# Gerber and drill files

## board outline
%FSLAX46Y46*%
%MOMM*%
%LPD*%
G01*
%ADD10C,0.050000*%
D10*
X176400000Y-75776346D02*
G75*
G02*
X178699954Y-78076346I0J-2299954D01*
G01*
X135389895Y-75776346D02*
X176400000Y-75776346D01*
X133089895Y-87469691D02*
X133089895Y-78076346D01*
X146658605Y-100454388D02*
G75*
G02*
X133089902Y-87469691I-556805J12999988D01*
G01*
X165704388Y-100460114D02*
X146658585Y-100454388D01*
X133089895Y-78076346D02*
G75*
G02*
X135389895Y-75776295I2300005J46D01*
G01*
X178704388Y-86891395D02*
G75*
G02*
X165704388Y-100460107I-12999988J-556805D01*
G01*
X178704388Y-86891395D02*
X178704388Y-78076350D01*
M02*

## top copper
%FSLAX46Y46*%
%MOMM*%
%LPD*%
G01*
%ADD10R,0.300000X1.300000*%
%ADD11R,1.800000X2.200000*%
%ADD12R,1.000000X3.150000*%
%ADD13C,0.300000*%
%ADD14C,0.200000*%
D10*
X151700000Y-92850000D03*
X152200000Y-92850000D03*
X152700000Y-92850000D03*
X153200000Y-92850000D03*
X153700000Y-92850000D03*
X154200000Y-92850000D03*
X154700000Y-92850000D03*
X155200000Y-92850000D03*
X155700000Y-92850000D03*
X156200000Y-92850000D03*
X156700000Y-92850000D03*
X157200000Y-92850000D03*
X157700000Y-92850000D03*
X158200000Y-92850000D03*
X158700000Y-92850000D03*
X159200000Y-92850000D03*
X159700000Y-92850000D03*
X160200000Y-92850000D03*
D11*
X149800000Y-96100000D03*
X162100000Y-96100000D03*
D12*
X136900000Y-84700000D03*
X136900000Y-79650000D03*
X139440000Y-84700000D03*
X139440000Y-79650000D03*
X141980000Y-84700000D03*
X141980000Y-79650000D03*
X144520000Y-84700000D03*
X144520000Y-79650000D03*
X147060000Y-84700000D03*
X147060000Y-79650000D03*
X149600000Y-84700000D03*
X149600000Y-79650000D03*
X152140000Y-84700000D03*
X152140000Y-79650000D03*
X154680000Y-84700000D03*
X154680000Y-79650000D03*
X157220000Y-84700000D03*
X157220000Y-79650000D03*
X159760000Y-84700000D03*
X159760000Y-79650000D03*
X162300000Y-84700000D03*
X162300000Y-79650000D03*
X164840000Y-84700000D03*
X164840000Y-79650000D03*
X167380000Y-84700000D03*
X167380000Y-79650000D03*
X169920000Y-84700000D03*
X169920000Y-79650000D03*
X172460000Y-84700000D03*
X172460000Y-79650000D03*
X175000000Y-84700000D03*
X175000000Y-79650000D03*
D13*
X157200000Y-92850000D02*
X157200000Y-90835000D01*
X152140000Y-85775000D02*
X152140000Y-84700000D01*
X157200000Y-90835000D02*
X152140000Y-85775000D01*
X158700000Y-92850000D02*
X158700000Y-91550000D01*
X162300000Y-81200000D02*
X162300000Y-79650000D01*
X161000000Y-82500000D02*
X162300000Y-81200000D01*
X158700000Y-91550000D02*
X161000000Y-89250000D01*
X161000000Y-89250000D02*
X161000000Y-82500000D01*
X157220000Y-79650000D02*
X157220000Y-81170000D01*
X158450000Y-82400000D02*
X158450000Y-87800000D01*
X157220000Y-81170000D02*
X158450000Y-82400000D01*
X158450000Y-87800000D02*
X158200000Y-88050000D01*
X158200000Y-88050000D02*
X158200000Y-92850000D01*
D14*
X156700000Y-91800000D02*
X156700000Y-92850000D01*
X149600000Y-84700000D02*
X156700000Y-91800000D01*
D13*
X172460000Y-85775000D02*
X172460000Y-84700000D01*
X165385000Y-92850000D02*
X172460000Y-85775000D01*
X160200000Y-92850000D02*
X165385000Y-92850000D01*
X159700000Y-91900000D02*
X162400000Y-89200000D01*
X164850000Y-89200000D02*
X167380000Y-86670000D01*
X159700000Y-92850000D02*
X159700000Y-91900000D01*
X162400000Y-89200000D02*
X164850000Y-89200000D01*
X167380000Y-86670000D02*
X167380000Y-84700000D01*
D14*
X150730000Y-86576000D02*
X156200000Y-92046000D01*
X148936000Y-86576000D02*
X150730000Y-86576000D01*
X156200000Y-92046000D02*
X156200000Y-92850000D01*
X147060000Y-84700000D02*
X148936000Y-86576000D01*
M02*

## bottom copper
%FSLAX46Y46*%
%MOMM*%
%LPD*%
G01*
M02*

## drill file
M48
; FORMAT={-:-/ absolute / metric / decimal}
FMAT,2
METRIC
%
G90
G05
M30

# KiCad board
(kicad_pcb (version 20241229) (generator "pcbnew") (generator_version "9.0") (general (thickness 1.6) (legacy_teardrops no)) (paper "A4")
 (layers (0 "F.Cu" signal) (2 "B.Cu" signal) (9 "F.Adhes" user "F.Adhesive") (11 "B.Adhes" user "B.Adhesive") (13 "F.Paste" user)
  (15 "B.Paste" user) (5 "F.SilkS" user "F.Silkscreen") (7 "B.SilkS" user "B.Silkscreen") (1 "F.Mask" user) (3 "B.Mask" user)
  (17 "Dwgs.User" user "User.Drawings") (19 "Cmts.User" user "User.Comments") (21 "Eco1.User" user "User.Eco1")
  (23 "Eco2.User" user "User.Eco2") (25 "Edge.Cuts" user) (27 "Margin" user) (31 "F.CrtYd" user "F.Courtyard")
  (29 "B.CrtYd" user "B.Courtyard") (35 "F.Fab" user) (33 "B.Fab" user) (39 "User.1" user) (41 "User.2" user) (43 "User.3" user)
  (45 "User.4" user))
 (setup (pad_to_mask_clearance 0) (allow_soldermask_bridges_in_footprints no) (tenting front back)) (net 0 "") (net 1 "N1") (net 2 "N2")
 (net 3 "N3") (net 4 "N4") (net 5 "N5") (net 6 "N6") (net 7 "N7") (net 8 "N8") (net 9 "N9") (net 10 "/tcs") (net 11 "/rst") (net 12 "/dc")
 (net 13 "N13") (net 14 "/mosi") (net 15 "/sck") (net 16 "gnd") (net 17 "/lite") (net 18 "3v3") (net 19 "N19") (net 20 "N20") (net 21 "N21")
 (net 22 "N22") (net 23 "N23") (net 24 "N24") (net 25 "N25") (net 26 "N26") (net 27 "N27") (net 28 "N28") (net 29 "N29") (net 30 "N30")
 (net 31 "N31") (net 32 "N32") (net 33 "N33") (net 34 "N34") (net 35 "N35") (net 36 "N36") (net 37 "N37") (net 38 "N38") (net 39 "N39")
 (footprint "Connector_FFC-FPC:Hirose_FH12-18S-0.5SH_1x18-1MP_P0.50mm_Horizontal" (layer "F.Cu") (at 155.95 94.7)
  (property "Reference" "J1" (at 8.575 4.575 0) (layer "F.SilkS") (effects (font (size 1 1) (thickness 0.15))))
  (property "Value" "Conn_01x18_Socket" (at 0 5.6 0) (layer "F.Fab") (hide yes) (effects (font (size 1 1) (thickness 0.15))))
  (pad "1" smd rect (at -4.25 -1.85) (size 0.3 1.3) (layers "F.Cu" "F.Mask" "F.Paste") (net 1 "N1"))
  (pad "2" smd rect (at -3.75 -1.85) (size 0.3 1.3) (layers "F.Cu" "F.Mask" "F.Paste") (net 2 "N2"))
  (pad "3" smd rect (at -3.25 -1.85) (size 0.3 1.3) (layers "F.Cu" "F.Mask" "F.Paste") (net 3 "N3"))
  (pad "4" smd rect (at -2.75 -1.85) (size 0.3 1.3) (layers "F.Cu" "F.Mask" "F.Paste") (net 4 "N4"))
  (pad "5" smd rect (at -2.25 -1.85) (size 0.3 1.3) (layers "F.Cu" "F.Mask" "F.Paste") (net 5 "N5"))
  (pad "6" smd rect (at -1.75 -1.85) (size 0.3 1.3) (layers "F.Cu" "F.Mask" "F.Paste") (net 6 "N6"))
  (pad "7" smd rect (at -1.25 -1.85) (size 0.3 1.3) (layers "F.Cu" "F.Mask" "F.Paste") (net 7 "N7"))
  (pad "8" smd rect (at -0.75 -1.85) (size 0.3 1.3) (layers "F.Cu" "F.Mask" "F.Paste") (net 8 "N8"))
  (pad "9" smd rect (at -0.25 -1.85) (size 0.3 1.3) (layers "F.Cu" "F.Mask" "F.Paste") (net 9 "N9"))
  (pad "10" smd rect (at 0.25 -1.85) (size 0.3 1.3) (layers "F.Cu" "F.Mask" "F.Paste") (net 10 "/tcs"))
  (pad "11" smd rect (at 0.75 -1.85) (size 0.3 1.3) (layers "F.Cu" "F.Mask" "F.Paste") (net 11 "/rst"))
  (pad "12" smd rect (at 1.25 -1.85) (size 0.3 1.3) (layers "F.Cu" "F.Mask" "F.Paste") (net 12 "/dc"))
  (pad "13" smd rect (at 1.75 -1.85) (size 0.3 1.3) (layers "F.Cu" "F.Mask" "F.Paste") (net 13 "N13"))
  (pad "14" smd rect (at 2.25 -1.85) (size 0.3 1.3) (layers "F.Cu" "F.Mask" "F.Paste") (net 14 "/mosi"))
  (pad "15" smd rect (at 2.75 -1.85) (size 0.3 1.3) (layers "F.Cu" "F.Mask" "F.Paste") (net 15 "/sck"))
  (pad "16" smd rect (at 3.25 -1.85) (size 0.3 1.3) (layers "F.Cu" "F.Mask" "F.Paste") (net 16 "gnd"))
  (pad "17" smd rect (at 3.75 -1.85) (size 0.3 1.3) (layers "F.Cu" "F.Mask" "F.Paste") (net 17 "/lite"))
  (pad "18" smd rect (at 4.25 -1.85) (size 0.3 1.3) (layers "F.Cu" "F.Mask" "F.Paste") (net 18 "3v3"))
  (pad "MP" smd rect (at -6.15 1.4) (size 1.8 2.2) (layers "F.Cu" "F.Mask" "F.Paste"))
  (pad "MP" smd rect (at 6.15 1.4) (size 1.8 2.2) (layers "F.Cu" "F.Mask" "F.Paste")))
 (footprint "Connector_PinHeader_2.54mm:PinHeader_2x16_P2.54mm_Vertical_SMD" (layer "F.Cu") (at 155.95 82.175 90)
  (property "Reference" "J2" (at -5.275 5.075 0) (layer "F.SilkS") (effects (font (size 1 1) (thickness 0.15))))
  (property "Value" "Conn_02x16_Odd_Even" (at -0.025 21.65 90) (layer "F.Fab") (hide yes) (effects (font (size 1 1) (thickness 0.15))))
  (pad "1" smd rect (at -2.525 -19.05 90) (size 3.15 1) (layers "F.Cu" "F.Mask" "F.Paste") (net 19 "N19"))
  (pad "2" smd rect (at 2.525 -19.05 90) (size 3.15 1) (layers "F.Cu" "F.Mask" "F.Paste") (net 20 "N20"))
  (pad "3" smd rect (at -2.525 -16.51 90) (size 3.15 1) (layers "F.Cu" "F.Mask" "F.Paste") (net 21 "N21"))
  (pad "4" smd rect (at 2.525 -16.51 90) (size 3.15 1) (layers "F.Cu" "F.Mask" "F.Paste") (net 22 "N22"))
  (pad "5" smd rect (at -2.525 -13.97 90) (size 3.15 1) (layers "F.Cu" "F.Mask" "F.Paste") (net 16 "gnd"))
  (pad "6" smd rect (at 2.525 -13.97 90) (size 3.15 1) (layers "F.Cu" "F.Mask" "F.Paste") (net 16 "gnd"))
  (pad "7" smd rect (at -2.525 -11.43 90) (size 3.15 1) (layers "F.Cu" "F.Mask" "F.Paste") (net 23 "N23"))
  (pad "8" smd rect (at 2.525 -11.43 90) (size 3.15 1) (layers "F.Cu" "F.Mask" "F.Paste") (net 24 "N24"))
  (pad "9" smd rect (at -2.525 -8.89 90) (size 3.15 1) (layers "F.Cu" "F.Mask" "F.Paste") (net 10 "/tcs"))
  (pad "10" smd rect (at 2.525 -8.89 90) (size 3.15 1) (layers "F.Cu" "F.Mask" "F.Paste") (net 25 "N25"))
  (pad "11" smd rect (at -2.525 -6.35 90) (size 3.15 1) (layers "F.Cu" "F.Mask" "F.Paste") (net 11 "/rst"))
  (pad "12" smd rect (at 2.525 -6.35 90) (size 3.15 1) (layers "F.Cu" "F.Mask" "F.Paste") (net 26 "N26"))
  (pad "13" smd rect (at -2.525 -3.81 90) (size 3.15 1) (layers "F.Cu" "F.Mask" "F.Paste") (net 12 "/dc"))
  (pad "14" smd rect (at 2.525 -3.81 90) (size 3.15 1) (layers "F.Cu" "F.Mask" "F.Paste") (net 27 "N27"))
  (pad "15" smd rect (at -2.525 -1.27 90) (size 3.15 1) (layers "F.Cu" "F.Mask" "F.Paste") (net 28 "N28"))
  (pad "16" smd rect (at 2.525 -1.27 90) (size 3.15 1) (layers "F.Cu" "F.Mask" "F.Paste") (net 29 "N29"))
  (pad "17" smd rect (at -2.525 1.27 90) (size 3.15 1) (layers "F.Cu" "F.Mask" "F.Paste") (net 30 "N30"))
  (pad "18" smd rect (at 2.525 1.27 90) (size 3.15 1) (layers "F.Cu" "F.Mask" "F.Paste") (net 14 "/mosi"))
  (pad "19" smd rect (at -2.525 3.81 90) (size 3.15 1) (layers "F.Cu" "F.Mask" "F.Paste") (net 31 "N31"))
  (pad "20" smd rect (at 2.525 3.81 90) (size 3.15 1) (layers "F.Cu" "F.Mask" "F.Paste") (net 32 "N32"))
  (pad "21" smd rect (at -2.525 6.35 90) (size 3.15 1) (layers "F.Cu" "F.Mask" "F.Paste") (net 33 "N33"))
  (pad "22" smd rect (at 2.525 6.35 90) (size 3.15 1) (layers "F.Cu" "F.Mask" "F.Paste") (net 15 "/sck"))
  (pad "23" smd rect (at -2.525 8.89 90) (size 3.15 1) (layers "F.Cu" "F.Mask" "F.Paste") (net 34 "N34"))
  (pad "24" smd rect (at 2.525 8.89 90) (size 3.15 1) (layers "F.Cu" "F.Mask" "F.Paste") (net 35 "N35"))
  (pad "25" smd rect (at -2.525 11.43 90) (size 3.15 1) (layers "F.Cu" "F.Mask" "F.Paste") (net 17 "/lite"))
  (pad "26" smd rect (at 2.525 11.43 90) (size 3.15 1) (layers "F.Cu" "F.Mask" "F.Paste") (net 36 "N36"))
  (pad "27" smd rect (at -2.525 13.97 90) (size 3.15 1) (layers "F.Cu" "F.Mask" "F.Paste") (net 16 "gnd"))
  (pad "28" smd rect (at 2.525 13.97 90) (size 3.15 1) (layers "F.Cu" "F.Mask" "F.Paste") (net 16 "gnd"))
  (pad "29" smd rect (at -2.525 16.51 90) (size 3.15 1) (layers "F.Cu" "F.Mask" "F.Paste") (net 18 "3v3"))
  (pad "30" smd rect (at 2.525 16.51 90) (size 3.15 1) (layers "F.Cu" "F.Mask" "F.Paste") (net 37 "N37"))
  (pad "31" smd rect (at -2.525 19.05 90) (size 3.15 1) (layers "F.Cu" "F.Mask" "F.Paste") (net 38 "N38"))
  (pad "32" smd rect (at 2.525 19.05 90) (size 3.15 1) (layers "F.Cu" "F.Mask" "F.Paste") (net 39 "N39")))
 (gr_arc (start 176.4 75.776346) (mid 178.026346 76.45) (end 178.7 78.076346) (stroke (width 0.05) (type default)) (layer "Edge.Cuts"))
 (gr_line (start 135.389895 75.776346) (end 176.4 75.776346) (stroke (width 0.05) (type default)) (layer "Edge.Cuts"))
 (gr_line (start 133.089895 87.469691) (end 133.089895 78.076346) (stroke (width 0.05) (type default)) (layer "Edge.Cuts"))
 (gr_arc (start 146.658605 100.454388) (mid 137.105527 96.855292) (end 133.089895 87.469691) (stroke (width 0.05) (type default))
  (layer "Edge.Cuts"))
 (gr_line (start 165.704388 100.460114) (end 146.658585 100.454388) (stroke (width 0.05) (type default)) (layer "Edge.Cuts"))
 (gr_arc (start 133.089895 78.076346) (mid 133.763549 76.45) (end 135.389895 75.776346) (stroke (width 0.05) (type default))
  (layer "Edge.Cuts"))
 (gr_arc (start 178.704388 86.891395) (mid 175.1 96.45) (end 165.704388 100.460114) (stroke (width 0.05) (type default)) (layer "Edge.Cuts"))
 (gr_line (start 178.704388 86.891395) (end 178.704388 78.07635) (stroke (width 0.05) (type default)) (layer "Edge.Cuts"))
 (segment (start 157.2 92.85) (end 157.2 90.835) (width 0.3) (layer "F.Cu") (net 12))
 (segment (start 152.14 85.775) (end 152.14 84.7) (width 0.3) (layer "F.Cu") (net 12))
 (segment (start 157.2 90.835) (end 152.14 85.775) (width 0.3) (layer "F.Cu") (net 12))
 (segment (start 158.7 92.85) (end 158.7 91.55) (width 0.3) (layer "F.Cu") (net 15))
 (segment (start 162.3 81.2) (end 162.3 79.65) (width 0.3) (layer "F.Cu") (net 15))
 (segment (start 161 82.5) (end 162.3 81.2) (width 0.3) (layer "F.Cu") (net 15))
 (segment (start 158.7 91.55) (end 161 89.25) (width 0.3) (layer "F.Cu") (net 15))
 (segment (start 161 89.25) (end 161 82.5) (width 0.3) (layer "F.Cu") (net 15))
 (segment (start 157.22 79.65) (end 157.22 81.17) (width 0.3) (layer "F.Cu") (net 14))
 (segment (start 158.45 82.4) (end 158.45 87.8) (width 0.3) (layer "F.Cu") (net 14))
 (segment (start 157.22 81.17) (end 158.45 82.4) (width 0.3) (layer "F.Cu") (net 14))
 (segment (start 158.45 87.8) (end 158.2 88.05) (width 0.3) (layer "F.Cu") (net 14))
 (segment (start 158.2 88.05) (end 158.2 92.85) (width 0.3) (layer "F.Cu") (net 14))
 (segment (start 156.7 91.8) (end 156.7 92.85) (width 0.2) (layer "F.Cu") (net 11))
 (segment (start 149.6 84.7) (end 156.7 91.8) (width 0.2) (layer "F.Cu") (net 11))
 (segment (start 172.46 85.775) (end 172.46 84.7) (width 0.3) (layer "F.Cu") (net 18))
 (segment (start 165.385 92.85) (end 172.46 85.775) (width 0.3) (layer "F.Cu") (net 18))
 (segment (start 160.2 92.85) (end 165.385 92.85) (width 0.3) (layer "F.Cu") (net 18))
 (segment (start 159.7 91.9) (end 162.4 89.2) (width 0.3) (layer "F.Cu") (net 17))
 (segment (start 164.85 89.2) (end 167.38 86.67) (width 0.3) (layer "F.Cu") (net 17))
 (segment (start 159.7 92.85) (end 159.7 91.9) (width 0.3) (layer "F.Cu") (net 17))
 (segment (start 162.4 89.2) (end 164.85 89.2) (width 0.3) (layer "F.Cu") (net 17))
 (segment (start 167.38 86.67) (end 167.38 84.7) (width 0.3) (layer "F.Cu") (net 17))
 (segment (start 150.73 86.576) (end 156.2 92.046) (width 0.2) (layer "F.Cu") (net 10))
 (segment (start 148.936 86.576) (end 150.73 86.576) (width 0.2) (layer "F.Cu") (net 10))
 (segment (start 156.2 92.046) (end 156.2 92.85) (width 0.2) (layer "F.Cu") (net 10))
 (segment (start 147.06 84.7) (end 148.936 86.576) (width 0.2) (layer "F.Cu") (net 10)))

